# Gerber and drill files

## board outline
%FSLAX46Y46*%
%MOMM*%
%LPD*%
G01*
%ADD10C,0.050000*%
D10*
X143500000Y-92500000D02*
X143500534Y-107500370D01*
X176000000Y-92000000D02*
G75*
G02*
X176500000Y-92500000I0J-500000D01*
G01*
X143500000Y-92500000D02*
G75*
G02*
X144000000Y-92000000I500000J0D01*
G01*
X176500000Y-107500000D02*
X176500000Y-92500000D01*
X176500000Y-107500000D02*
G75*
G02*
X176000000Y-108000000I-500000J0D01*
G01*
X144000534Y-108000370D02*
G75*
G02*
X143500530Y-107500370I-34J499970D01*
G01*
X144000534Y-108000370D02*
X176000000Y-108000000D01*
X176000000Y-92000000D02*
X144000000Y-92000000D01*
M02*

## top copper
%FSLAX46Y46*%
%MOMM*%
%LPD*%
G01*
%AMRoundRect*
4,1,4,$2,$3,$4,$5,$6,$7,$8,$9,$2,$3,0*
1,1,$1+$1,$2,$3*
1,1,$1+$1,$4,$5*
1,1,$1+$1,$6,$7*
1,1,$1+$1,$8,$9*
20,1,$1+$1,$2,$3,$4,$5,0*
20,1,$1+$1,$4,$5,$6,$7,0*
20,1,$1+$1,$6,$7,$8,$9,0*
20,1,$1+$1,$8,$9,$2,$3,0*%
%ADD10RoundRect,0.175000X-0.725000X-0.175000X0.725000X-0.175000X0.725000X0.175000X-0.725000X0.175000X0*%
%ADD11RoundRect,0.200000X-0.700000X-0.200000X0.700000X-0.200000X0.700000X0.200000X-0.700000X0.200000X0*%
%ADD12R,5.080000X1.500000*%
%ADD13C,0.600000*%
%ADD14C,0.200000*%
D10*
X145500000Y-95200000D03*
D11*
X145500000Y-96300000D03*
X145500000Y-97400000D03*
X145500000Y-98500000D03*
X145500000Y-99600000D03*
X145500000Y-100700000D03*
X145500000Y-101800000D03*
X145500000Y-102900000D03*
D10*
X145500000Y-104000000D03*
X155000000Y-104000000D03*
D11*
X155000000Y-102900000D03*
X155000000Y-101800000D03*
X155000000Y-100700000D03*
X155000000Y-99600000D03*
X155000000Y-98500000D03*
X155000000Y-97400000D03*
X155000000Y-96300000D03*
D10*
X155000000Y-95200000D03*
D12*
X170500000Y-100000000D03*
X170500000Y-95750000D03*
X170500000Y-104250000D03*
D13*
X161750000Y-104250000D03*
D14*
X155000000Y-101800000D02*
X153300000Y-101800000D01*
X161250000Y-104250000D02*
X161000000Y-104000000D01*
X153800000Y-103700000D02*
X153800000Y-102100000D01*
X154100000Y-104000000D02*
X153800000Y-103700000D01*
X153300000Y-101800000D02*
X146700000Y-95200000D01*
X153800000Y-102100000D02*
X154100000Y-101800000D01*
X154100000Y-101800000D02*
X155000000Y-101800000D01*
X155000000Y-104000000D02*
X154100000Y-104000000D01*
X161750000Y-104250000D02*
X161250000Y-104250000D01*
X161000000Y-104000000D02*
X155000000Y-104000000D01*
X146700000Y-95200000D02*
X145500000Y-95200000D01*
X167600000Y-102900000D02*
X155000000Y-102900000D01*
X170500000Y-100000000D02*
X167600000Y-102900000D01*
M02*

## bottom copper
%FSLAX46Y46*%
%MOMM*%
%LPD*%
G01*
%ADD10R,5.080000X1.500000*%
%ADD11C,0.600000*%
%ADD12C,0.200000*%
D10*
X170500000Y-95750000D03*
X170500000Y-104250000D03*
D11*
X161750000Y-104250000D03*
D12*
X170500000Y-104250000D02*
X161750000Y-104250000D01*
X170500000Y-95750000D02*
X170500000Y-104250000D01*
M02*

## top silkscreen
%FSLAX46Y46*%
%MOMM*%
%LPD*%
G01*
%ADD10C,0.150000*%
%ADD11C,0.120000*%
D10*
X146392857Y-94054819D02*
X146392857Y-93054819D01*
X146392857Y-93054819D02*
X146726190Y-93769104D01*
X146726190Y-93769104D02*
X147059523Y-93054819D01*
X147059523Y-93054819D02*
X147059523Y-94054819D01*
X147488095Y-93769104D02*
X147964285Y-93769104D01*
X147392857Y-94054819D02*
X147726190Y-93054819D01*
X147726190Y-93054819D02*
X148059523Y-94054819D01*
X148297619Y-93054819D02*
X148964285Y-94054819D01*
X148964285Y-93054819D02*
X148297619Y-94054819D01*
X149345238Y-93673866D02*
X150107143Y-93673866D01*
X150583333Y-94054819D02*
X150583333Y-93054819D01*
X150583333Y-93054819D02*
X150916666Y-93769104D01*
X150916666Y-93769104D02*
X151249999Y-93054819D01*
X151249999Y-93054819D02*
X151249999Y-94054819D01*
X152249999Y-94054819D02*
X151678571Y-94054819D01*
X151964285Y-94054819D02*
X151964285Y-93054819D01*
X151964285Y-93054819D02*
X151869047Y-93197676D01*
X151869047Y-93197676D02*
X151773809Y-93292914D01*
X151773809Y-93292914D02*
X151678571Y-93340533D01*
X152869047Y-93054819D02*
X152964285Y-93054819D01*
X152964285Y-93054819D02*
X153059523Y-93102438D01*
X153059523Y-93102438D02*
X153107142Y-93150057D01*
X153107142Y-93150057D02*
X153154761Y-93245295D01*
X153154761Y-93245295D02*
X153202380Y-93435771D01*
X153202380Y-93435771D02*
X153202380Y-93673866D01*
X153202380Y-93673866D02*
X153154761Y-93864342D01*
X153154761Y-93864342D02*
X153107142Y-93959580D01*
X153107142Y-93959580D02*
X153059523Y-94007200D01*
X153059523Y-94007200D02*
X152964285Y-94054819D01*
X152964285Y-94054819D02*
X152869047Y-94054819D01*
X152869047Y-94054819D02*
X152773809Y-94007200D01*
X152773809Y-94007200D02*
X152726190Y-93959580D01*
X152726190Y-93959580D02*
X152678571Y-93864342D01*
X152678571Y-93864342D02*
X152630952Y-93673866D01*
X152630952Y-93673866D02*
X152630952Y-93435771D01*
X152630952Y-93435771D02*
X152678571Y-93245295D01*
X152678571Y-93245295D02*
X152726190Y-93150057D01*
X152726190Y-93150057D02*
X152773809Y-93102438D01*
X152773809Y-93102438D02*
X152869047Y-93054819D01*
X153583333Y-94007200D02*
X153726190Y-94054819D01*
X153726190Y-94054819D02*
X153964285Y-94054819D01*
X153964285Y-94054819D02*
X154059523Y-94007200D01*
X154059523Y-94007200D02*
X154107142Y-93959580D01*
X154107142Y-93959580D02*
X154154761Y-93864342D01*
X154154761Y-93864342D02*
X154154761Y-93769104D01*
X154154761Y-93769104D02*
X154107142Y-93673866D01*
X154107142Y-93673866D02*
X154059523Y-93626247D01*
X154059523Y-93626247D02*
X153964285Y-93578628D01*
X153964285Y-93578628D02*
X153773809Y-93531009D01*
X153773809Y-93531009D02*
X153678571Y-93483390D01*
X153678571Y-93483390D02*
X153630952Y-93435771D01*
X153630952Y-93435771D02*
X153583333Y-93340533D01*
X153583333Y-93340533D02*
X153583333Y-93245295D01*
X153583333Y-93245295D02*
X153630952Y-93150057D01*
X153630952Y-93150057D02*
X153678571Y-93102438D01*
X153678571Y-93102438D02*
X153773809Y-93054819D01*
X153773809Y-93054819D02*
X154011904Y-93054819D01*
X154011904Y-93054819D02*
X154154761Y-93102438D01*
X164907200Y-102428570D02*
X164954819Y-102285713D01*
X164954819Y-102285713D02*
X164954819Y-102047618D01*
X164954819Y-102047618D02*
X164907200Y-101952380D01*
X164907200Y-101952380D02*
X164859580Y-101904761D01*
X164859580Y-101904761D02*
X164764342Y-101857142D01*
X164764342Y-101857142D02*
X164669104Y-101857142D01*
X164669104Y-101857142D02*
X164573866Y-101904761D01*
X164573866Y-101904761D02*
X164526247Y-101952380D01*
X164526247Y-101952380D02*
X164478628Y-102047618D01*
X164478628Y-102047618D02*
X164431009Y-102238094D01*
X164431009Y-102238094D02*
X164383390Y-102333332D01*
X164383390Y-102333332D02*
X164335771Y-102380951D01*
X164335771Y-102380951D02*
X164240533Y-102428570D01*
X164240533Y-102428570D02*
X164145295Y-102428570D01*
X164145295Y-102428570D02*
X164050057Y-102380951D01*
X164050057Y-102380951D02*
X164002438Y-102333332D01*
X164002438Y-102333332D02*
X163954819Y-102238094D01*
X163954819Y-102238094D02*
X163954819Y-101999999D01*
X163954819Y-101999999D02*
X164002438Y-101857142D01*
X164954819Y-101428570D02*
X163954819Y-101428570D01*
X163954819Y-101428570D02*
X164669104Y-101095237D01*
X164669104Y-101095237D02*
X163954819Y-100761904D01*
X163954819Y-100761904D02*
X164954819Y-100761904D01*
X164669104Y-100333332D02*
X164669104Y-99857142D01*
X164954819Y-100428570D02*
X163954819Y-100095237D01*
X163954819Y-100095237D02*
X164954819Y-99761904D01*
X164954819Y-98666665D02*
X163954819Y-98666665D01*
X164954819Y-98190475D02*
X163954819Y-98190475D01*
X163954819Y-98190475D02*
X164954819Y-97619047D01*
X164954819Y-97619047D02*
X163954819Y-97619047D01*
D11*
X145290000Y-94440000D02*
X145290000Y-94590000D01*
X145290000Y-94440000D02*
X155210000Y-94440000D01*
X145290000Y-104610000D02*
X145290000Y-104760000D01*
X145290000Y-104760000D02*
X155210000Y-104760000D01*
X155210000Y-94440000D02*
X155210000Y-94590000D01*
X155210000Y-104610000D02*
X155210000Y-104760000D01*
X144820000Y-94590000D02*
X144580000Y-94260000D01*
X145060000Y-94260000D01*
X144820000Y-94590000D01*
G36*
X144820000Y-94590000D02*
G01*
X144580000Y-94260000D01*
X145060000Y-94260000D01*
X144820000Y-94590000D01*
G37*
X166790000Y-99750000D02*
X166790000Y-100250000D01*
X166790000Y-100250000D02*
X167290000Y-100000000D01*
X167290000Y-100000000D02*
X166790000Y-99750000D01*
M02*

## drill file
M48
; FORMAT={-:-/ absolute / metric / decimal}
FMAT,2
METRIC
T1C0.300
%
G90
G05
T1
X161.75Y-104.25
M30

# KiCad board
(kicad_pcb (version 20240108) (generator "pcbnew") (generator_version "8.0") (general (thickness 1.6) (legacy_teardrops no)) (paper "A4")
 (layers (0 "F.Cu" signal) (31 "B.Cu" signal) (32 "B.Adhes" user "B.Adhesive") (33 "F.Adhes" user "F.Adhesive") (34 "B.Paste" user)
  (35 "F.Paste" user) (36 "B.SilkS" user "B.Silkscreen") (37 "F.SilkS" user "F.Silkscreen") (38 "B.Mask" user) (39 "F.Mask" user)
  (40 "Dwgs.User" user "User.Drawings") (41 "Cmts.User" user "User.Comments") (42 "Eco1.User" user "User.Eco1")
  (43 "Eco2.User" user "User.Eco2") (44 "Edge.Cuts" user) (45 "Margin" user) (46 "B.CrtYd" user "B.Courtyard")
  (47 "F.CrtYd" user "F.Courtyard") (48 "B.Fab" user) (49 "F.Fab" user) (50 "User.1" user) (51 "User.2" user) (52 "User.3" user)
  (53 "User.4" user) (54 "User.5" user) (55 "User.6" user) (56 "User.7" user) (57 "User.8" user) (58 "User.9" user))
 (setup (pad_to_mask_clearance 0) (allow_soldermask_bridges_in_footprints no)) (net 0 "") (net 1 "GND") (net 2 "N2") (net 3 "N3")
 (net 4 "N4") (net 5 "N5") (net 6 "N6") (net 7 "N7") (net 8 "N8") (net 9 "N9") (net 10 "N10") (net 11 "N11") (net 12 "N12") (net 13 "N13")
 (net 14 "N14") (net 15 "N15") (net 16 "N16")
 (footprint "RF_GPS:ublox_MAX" (layer "F.Cu") (at 150.25 99.6)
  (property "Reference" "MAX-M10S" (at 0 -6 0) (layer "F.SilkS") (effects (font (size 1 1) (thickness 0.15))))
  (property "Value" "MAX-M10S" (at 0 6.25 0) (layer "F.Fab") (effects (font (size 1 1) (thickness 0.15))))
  (fp_line (start -4.96 -5.16) (end -4.96 -5.01) (stroke (width 0.12) (type solid)) (layer "F.SilkS"))
  (fp_line (start -4.96 -5.16) (end 4.96 -5.16) (stroke (width 0.12) (type solid)) (layer "F.SilkS"))
  (fp_line (start -4.96 5.01) (end -4.96 5.16) (stroke (width 0.12) (type solid)) (layer "F.SilkS"))
  (fp_line (start -4.96 5.16) (end 4.96 5.16) (stroke (width 0.12) (type solid)) (layer "F.SilkS"))
  (fp_line (start 4.96 -5.16) (end 4.96 -5.01) (stroke (width 0.12) (type solid)) (layer "F.SilkS"))
  (fp_line (start 4.96 5.01) (end 4.96 5.16) (stroke (width 0.12) (type solid)) (layer "F.SilkS"))
  (fp_poly
   (pts (xy -5.43 -5.01) (xy -5.67 -5.34) (xy -5.19 -5.34) (xy -5.43 -5.01)) (stroke (width 0.12) (type solid)) (fill solid)
   (layer "F.SilkS"))
  (pad "1" smd roundrect (at -4.75 -4.4) (size 1.8 0.7) (layers "F.Cu" "F.Paste" "F.Mask") (roundrect_rratio 0.25) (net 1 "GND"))
  (pad "2" smd roundrect (at -4.75 -3.3) (size 1.8 0.8) (layers "F.Cu" "F.Paste" "F.Mask") (roundrect_rratio 0.25) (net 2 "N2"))
  (pad "3" smd roundrect (at -4.75 -2.2) (size 1.8 0.8) (layers "F.Cu" "F.Paste" "F.Mask") (roundrect_rratio 0.25) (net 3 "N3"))
  (pad "4" smd roundrect (at -4.75 -1.1) (size 1.8 0.8) (layers "F.Cu" "F.Paste" "F.Mask") (roundrect_rratio 0.25) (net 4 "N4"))
  (pad "5" smd roundrect (at -4.75 0) (size 1.8 0.8) (layers "F.Cu" "F.Paste" "F.Mask") (roundrect_rratio 0.25) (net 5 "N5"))
  (pad "6" smd roundrect (at -4.75 1.1) (size 1.8 0.8) (layers "F.Cu" "F.Paste" "F.Mask") (roundrect_rratio 0.25) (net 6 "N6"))
  (pad "7" smd roundrect (at -4.75 2.2) (size 1.8 0.8) (layers "F.Cu" "F.Paste" "F.Mask") (roundrect_rratio 0.25) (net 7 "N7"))
  (pad "8" smd roundrect (at -4.75 3.3) (size 1.8 0.8) (layers "F.Cu" "F.Paste" "F.Mask") (roundrect_rratio 0.25) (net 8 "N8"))
  (pad "9" smd roundrect (at -4.75 4.4) (size 1.8 0.7) (layers "F.Cu" "F.Paste" "F.Mask") (roundrect_rratio 0.25) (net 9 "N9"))
  (pad "10" smd roundrect (at 4.75 4.4) (size 1.8 0.7) (layers "F.Cu" "F.Paste" "F.Mask") (roundrect_rratio 0.25) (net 1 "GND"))
  (pad "11" smd roundrect (at 4.75 3.3) (size 1.8 0.8) (layers "F.Cu" "F.Paste" "F.Mask") (roundrect_rratio 0.25) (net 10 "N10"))
  (pad "12" smd roundrect (at 4.75 2.2) (size 1.8 0.8) (layers "F.Cu" "F.Paste" "F.Mask") (roundrect_rratio 0.25) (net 1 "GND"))
  (pad "13" smd roundrect (at 4.75 1.1) (size 1.8 0.8) (layers "F.Cu" "F.Paste" "F.Mask") (roundrect_rratio 0.25) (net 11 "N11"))
  (pad "14" smd roundrect (at 4.75 0) (size 1.8 0.8) (layers "F.Cu" "F.Paste" "F.Mask") (roundrect_rratio 0.25) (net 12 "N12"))
  (pad "15" smd roundrect (at 4.75 -1.1) (size 1.8 0.8) (layers "F.Cu" "F.Paste" "F.Mask") (roundrect_rratio 0.25) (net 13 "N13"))
  (pad "16" smd roundrect (at 4.75 -2.2) (size 1.8 0.8) (layers "F.Cu" "F.Paste" "F.Mask") (roundrect_rratio 0.25) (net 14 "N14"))
  (pad "17" smd roundrect (at 4.75 -3.3) (size 1.8 0.8) (layers "F.Cu" "F.Paste" "F.Mask") (roundrect_rratio 0.25) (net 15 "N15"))
  (pad "18" smd roundrect (at 4.75 -4.4) (size 1.8 0.7) (layers "F.Cu" "F.Paste" "F.Mask") (roundrect_rratio 0.25) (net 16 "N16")))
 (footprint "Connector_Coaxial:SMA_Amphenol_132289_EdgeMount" (layer "F.Cu") (at 170.5 100)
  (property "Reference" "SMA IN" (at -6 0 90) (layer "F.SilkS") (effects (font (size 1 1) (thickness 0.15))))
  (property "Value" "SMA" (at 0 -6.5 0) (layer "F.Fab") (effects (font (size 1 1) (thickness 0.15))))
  (fp_line (start -3.71 -0.25) (end -3.71 0.25) (stroke (width 0.12) (type solid)) (layer "F.SilkS"))
  (fp_line (start -3.71 0.25) (end -3.21 0) (stroke (width 0.12) (type solid)) (layer "F.SilkS"))
  (fp_line (start -3.21 0) (end -3.71 -0.25) (stroke (width 0.12) (type solid)) (layer "F.SilkS"))
  (pad "1" smd rect (at 0 0 90) (size 1.5 5.08) (layers "F.Cu" "F.Paste" "F.Mask") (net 10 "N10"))
  (pad "2" smd rect (at 0 -4.25 90) (size 1.5 5.08) (layers "F.Cu" "F.Paste" "F.Mask") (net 1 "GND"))
  (pad "2" smd rect (at 0 -4.25 90) (size 1.5 5.08) (layers "B.Cu" "B.Paste" "B.Mask") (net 1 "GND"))
  (pad "2" smd rect (at 0 4.25 90) (size 1.5 5.08) (layers "F.Cu" "F.Paste" "F.Mask") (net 1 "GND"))
  (pad "2" smd rect (at 0 4.25 90) (size 1.5 5.08) (layers "B.Cu" "B.Paste" "B.Mask") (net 1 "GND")))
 (gr_line (start 143.5 92.5) (end 143.500534 107.50037) (stroke (width 0.05) (type default)) (layer "Edge.Cuts"))
 (gr_arc (start 176 92) (mid 176.353553 92.146447) (end 176.5 92.5) (stroke (width 0.05) (type default)) (layer "Edge.Cuts"))
 (gr_arc (start 143.5 92.5) (mid 143.646447 92.146447) (end 144 92) (stroke (width 0.05) (type default)) (layer "Edge.Cuts"))
 (gr_line (start 176.5 107.5) (end 176.5 92.5) (stroke (width 0.05) (type default)) (layer "Edge.Cuts"))
 (gr_arc (start 176.5 107.5) (mid 176.353553 107.853553) (end 176 108) (stroke (width 0.05) (type default)) (layer "Edge.Cuts"))
 (gr_arc (start 144.000534 108.00037) (mid 143.646981 107.853923) (end 143.500534 107.50037) (stroke (width 0.05) (type default))
  (layer "Edge.Cuts"))
 (gr_line (start 144.000534 108.00037) (end 176 108) (stroke (width 0.05) (type default)) (layer "Edge.Cuts"))
 (gr_line (start 176 92) (end 144 92) (stroke (width 0.05) (type default)) (layer "Edge.Cuts"))
 (segment (start 155 101.8) (end 153.3 101.8) (width 0.2) (layer "F.Cu") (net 1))
 (segment (start 161.25 104.25) (end 161 104) (width 0.2) (layer "F.Cu") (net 1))
 (segment (start 153.8 103.7) (end 153.8 102.1) (width 0.2) (layer "F.Cu") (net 1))
 (segment (start 154.1 104) (end 153.8 103.7) (width 0.2) (layer "F.Cu") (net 1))
 (segment (start 153.3 101.8) (end 146.7 95.2) (width 0.2) (layer "F.Cu") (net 1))
 (segment (start 153.8 102.1) (end 154.1 101.8) (width 0.2) (layer "F.Cu") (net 1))
 (segment (start 154.1 101.8) (end 155 101.8) (width 0.2) (layer "F.Cu") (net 1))
 (segment (start 155 104) (end 154.1 104) (width 0.2) (layer "F.Cu") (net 1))
 (segment (start 161.75 104.25) (end 161.25 104.25) (width 0.2) (layer "F.Cu") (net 1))
 (segment (start 161 104) (end 155 104) (width 0.2) (layer "F.Cu") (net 1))
 (segment (start 146.7 95.2) (end 145.5 95.2) (width 0.2) (layer "F.Cu") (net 1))
 (via (at 161.75 104.25) (size 0.6) (drill 0.3) (layers "F.Cu" "B.Cu") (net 1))
 (segment (start 170.5 104.25) (end 161.75 104.25) (width 0.2) (layer "B.Cu") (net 1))
 (segment (start 170.5 95.75) (end 170.5 104.25) (width 0.2) (layer "B.Cu") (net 1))
 (segment (start 167.6 102.9) (end 155 102.9) (width 0.2) (layer "F.Cu") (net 10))
 (segment (start 170.5 100) (end 167.6 102.9) (width 0.2) (layer "F.Cu") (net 10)))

